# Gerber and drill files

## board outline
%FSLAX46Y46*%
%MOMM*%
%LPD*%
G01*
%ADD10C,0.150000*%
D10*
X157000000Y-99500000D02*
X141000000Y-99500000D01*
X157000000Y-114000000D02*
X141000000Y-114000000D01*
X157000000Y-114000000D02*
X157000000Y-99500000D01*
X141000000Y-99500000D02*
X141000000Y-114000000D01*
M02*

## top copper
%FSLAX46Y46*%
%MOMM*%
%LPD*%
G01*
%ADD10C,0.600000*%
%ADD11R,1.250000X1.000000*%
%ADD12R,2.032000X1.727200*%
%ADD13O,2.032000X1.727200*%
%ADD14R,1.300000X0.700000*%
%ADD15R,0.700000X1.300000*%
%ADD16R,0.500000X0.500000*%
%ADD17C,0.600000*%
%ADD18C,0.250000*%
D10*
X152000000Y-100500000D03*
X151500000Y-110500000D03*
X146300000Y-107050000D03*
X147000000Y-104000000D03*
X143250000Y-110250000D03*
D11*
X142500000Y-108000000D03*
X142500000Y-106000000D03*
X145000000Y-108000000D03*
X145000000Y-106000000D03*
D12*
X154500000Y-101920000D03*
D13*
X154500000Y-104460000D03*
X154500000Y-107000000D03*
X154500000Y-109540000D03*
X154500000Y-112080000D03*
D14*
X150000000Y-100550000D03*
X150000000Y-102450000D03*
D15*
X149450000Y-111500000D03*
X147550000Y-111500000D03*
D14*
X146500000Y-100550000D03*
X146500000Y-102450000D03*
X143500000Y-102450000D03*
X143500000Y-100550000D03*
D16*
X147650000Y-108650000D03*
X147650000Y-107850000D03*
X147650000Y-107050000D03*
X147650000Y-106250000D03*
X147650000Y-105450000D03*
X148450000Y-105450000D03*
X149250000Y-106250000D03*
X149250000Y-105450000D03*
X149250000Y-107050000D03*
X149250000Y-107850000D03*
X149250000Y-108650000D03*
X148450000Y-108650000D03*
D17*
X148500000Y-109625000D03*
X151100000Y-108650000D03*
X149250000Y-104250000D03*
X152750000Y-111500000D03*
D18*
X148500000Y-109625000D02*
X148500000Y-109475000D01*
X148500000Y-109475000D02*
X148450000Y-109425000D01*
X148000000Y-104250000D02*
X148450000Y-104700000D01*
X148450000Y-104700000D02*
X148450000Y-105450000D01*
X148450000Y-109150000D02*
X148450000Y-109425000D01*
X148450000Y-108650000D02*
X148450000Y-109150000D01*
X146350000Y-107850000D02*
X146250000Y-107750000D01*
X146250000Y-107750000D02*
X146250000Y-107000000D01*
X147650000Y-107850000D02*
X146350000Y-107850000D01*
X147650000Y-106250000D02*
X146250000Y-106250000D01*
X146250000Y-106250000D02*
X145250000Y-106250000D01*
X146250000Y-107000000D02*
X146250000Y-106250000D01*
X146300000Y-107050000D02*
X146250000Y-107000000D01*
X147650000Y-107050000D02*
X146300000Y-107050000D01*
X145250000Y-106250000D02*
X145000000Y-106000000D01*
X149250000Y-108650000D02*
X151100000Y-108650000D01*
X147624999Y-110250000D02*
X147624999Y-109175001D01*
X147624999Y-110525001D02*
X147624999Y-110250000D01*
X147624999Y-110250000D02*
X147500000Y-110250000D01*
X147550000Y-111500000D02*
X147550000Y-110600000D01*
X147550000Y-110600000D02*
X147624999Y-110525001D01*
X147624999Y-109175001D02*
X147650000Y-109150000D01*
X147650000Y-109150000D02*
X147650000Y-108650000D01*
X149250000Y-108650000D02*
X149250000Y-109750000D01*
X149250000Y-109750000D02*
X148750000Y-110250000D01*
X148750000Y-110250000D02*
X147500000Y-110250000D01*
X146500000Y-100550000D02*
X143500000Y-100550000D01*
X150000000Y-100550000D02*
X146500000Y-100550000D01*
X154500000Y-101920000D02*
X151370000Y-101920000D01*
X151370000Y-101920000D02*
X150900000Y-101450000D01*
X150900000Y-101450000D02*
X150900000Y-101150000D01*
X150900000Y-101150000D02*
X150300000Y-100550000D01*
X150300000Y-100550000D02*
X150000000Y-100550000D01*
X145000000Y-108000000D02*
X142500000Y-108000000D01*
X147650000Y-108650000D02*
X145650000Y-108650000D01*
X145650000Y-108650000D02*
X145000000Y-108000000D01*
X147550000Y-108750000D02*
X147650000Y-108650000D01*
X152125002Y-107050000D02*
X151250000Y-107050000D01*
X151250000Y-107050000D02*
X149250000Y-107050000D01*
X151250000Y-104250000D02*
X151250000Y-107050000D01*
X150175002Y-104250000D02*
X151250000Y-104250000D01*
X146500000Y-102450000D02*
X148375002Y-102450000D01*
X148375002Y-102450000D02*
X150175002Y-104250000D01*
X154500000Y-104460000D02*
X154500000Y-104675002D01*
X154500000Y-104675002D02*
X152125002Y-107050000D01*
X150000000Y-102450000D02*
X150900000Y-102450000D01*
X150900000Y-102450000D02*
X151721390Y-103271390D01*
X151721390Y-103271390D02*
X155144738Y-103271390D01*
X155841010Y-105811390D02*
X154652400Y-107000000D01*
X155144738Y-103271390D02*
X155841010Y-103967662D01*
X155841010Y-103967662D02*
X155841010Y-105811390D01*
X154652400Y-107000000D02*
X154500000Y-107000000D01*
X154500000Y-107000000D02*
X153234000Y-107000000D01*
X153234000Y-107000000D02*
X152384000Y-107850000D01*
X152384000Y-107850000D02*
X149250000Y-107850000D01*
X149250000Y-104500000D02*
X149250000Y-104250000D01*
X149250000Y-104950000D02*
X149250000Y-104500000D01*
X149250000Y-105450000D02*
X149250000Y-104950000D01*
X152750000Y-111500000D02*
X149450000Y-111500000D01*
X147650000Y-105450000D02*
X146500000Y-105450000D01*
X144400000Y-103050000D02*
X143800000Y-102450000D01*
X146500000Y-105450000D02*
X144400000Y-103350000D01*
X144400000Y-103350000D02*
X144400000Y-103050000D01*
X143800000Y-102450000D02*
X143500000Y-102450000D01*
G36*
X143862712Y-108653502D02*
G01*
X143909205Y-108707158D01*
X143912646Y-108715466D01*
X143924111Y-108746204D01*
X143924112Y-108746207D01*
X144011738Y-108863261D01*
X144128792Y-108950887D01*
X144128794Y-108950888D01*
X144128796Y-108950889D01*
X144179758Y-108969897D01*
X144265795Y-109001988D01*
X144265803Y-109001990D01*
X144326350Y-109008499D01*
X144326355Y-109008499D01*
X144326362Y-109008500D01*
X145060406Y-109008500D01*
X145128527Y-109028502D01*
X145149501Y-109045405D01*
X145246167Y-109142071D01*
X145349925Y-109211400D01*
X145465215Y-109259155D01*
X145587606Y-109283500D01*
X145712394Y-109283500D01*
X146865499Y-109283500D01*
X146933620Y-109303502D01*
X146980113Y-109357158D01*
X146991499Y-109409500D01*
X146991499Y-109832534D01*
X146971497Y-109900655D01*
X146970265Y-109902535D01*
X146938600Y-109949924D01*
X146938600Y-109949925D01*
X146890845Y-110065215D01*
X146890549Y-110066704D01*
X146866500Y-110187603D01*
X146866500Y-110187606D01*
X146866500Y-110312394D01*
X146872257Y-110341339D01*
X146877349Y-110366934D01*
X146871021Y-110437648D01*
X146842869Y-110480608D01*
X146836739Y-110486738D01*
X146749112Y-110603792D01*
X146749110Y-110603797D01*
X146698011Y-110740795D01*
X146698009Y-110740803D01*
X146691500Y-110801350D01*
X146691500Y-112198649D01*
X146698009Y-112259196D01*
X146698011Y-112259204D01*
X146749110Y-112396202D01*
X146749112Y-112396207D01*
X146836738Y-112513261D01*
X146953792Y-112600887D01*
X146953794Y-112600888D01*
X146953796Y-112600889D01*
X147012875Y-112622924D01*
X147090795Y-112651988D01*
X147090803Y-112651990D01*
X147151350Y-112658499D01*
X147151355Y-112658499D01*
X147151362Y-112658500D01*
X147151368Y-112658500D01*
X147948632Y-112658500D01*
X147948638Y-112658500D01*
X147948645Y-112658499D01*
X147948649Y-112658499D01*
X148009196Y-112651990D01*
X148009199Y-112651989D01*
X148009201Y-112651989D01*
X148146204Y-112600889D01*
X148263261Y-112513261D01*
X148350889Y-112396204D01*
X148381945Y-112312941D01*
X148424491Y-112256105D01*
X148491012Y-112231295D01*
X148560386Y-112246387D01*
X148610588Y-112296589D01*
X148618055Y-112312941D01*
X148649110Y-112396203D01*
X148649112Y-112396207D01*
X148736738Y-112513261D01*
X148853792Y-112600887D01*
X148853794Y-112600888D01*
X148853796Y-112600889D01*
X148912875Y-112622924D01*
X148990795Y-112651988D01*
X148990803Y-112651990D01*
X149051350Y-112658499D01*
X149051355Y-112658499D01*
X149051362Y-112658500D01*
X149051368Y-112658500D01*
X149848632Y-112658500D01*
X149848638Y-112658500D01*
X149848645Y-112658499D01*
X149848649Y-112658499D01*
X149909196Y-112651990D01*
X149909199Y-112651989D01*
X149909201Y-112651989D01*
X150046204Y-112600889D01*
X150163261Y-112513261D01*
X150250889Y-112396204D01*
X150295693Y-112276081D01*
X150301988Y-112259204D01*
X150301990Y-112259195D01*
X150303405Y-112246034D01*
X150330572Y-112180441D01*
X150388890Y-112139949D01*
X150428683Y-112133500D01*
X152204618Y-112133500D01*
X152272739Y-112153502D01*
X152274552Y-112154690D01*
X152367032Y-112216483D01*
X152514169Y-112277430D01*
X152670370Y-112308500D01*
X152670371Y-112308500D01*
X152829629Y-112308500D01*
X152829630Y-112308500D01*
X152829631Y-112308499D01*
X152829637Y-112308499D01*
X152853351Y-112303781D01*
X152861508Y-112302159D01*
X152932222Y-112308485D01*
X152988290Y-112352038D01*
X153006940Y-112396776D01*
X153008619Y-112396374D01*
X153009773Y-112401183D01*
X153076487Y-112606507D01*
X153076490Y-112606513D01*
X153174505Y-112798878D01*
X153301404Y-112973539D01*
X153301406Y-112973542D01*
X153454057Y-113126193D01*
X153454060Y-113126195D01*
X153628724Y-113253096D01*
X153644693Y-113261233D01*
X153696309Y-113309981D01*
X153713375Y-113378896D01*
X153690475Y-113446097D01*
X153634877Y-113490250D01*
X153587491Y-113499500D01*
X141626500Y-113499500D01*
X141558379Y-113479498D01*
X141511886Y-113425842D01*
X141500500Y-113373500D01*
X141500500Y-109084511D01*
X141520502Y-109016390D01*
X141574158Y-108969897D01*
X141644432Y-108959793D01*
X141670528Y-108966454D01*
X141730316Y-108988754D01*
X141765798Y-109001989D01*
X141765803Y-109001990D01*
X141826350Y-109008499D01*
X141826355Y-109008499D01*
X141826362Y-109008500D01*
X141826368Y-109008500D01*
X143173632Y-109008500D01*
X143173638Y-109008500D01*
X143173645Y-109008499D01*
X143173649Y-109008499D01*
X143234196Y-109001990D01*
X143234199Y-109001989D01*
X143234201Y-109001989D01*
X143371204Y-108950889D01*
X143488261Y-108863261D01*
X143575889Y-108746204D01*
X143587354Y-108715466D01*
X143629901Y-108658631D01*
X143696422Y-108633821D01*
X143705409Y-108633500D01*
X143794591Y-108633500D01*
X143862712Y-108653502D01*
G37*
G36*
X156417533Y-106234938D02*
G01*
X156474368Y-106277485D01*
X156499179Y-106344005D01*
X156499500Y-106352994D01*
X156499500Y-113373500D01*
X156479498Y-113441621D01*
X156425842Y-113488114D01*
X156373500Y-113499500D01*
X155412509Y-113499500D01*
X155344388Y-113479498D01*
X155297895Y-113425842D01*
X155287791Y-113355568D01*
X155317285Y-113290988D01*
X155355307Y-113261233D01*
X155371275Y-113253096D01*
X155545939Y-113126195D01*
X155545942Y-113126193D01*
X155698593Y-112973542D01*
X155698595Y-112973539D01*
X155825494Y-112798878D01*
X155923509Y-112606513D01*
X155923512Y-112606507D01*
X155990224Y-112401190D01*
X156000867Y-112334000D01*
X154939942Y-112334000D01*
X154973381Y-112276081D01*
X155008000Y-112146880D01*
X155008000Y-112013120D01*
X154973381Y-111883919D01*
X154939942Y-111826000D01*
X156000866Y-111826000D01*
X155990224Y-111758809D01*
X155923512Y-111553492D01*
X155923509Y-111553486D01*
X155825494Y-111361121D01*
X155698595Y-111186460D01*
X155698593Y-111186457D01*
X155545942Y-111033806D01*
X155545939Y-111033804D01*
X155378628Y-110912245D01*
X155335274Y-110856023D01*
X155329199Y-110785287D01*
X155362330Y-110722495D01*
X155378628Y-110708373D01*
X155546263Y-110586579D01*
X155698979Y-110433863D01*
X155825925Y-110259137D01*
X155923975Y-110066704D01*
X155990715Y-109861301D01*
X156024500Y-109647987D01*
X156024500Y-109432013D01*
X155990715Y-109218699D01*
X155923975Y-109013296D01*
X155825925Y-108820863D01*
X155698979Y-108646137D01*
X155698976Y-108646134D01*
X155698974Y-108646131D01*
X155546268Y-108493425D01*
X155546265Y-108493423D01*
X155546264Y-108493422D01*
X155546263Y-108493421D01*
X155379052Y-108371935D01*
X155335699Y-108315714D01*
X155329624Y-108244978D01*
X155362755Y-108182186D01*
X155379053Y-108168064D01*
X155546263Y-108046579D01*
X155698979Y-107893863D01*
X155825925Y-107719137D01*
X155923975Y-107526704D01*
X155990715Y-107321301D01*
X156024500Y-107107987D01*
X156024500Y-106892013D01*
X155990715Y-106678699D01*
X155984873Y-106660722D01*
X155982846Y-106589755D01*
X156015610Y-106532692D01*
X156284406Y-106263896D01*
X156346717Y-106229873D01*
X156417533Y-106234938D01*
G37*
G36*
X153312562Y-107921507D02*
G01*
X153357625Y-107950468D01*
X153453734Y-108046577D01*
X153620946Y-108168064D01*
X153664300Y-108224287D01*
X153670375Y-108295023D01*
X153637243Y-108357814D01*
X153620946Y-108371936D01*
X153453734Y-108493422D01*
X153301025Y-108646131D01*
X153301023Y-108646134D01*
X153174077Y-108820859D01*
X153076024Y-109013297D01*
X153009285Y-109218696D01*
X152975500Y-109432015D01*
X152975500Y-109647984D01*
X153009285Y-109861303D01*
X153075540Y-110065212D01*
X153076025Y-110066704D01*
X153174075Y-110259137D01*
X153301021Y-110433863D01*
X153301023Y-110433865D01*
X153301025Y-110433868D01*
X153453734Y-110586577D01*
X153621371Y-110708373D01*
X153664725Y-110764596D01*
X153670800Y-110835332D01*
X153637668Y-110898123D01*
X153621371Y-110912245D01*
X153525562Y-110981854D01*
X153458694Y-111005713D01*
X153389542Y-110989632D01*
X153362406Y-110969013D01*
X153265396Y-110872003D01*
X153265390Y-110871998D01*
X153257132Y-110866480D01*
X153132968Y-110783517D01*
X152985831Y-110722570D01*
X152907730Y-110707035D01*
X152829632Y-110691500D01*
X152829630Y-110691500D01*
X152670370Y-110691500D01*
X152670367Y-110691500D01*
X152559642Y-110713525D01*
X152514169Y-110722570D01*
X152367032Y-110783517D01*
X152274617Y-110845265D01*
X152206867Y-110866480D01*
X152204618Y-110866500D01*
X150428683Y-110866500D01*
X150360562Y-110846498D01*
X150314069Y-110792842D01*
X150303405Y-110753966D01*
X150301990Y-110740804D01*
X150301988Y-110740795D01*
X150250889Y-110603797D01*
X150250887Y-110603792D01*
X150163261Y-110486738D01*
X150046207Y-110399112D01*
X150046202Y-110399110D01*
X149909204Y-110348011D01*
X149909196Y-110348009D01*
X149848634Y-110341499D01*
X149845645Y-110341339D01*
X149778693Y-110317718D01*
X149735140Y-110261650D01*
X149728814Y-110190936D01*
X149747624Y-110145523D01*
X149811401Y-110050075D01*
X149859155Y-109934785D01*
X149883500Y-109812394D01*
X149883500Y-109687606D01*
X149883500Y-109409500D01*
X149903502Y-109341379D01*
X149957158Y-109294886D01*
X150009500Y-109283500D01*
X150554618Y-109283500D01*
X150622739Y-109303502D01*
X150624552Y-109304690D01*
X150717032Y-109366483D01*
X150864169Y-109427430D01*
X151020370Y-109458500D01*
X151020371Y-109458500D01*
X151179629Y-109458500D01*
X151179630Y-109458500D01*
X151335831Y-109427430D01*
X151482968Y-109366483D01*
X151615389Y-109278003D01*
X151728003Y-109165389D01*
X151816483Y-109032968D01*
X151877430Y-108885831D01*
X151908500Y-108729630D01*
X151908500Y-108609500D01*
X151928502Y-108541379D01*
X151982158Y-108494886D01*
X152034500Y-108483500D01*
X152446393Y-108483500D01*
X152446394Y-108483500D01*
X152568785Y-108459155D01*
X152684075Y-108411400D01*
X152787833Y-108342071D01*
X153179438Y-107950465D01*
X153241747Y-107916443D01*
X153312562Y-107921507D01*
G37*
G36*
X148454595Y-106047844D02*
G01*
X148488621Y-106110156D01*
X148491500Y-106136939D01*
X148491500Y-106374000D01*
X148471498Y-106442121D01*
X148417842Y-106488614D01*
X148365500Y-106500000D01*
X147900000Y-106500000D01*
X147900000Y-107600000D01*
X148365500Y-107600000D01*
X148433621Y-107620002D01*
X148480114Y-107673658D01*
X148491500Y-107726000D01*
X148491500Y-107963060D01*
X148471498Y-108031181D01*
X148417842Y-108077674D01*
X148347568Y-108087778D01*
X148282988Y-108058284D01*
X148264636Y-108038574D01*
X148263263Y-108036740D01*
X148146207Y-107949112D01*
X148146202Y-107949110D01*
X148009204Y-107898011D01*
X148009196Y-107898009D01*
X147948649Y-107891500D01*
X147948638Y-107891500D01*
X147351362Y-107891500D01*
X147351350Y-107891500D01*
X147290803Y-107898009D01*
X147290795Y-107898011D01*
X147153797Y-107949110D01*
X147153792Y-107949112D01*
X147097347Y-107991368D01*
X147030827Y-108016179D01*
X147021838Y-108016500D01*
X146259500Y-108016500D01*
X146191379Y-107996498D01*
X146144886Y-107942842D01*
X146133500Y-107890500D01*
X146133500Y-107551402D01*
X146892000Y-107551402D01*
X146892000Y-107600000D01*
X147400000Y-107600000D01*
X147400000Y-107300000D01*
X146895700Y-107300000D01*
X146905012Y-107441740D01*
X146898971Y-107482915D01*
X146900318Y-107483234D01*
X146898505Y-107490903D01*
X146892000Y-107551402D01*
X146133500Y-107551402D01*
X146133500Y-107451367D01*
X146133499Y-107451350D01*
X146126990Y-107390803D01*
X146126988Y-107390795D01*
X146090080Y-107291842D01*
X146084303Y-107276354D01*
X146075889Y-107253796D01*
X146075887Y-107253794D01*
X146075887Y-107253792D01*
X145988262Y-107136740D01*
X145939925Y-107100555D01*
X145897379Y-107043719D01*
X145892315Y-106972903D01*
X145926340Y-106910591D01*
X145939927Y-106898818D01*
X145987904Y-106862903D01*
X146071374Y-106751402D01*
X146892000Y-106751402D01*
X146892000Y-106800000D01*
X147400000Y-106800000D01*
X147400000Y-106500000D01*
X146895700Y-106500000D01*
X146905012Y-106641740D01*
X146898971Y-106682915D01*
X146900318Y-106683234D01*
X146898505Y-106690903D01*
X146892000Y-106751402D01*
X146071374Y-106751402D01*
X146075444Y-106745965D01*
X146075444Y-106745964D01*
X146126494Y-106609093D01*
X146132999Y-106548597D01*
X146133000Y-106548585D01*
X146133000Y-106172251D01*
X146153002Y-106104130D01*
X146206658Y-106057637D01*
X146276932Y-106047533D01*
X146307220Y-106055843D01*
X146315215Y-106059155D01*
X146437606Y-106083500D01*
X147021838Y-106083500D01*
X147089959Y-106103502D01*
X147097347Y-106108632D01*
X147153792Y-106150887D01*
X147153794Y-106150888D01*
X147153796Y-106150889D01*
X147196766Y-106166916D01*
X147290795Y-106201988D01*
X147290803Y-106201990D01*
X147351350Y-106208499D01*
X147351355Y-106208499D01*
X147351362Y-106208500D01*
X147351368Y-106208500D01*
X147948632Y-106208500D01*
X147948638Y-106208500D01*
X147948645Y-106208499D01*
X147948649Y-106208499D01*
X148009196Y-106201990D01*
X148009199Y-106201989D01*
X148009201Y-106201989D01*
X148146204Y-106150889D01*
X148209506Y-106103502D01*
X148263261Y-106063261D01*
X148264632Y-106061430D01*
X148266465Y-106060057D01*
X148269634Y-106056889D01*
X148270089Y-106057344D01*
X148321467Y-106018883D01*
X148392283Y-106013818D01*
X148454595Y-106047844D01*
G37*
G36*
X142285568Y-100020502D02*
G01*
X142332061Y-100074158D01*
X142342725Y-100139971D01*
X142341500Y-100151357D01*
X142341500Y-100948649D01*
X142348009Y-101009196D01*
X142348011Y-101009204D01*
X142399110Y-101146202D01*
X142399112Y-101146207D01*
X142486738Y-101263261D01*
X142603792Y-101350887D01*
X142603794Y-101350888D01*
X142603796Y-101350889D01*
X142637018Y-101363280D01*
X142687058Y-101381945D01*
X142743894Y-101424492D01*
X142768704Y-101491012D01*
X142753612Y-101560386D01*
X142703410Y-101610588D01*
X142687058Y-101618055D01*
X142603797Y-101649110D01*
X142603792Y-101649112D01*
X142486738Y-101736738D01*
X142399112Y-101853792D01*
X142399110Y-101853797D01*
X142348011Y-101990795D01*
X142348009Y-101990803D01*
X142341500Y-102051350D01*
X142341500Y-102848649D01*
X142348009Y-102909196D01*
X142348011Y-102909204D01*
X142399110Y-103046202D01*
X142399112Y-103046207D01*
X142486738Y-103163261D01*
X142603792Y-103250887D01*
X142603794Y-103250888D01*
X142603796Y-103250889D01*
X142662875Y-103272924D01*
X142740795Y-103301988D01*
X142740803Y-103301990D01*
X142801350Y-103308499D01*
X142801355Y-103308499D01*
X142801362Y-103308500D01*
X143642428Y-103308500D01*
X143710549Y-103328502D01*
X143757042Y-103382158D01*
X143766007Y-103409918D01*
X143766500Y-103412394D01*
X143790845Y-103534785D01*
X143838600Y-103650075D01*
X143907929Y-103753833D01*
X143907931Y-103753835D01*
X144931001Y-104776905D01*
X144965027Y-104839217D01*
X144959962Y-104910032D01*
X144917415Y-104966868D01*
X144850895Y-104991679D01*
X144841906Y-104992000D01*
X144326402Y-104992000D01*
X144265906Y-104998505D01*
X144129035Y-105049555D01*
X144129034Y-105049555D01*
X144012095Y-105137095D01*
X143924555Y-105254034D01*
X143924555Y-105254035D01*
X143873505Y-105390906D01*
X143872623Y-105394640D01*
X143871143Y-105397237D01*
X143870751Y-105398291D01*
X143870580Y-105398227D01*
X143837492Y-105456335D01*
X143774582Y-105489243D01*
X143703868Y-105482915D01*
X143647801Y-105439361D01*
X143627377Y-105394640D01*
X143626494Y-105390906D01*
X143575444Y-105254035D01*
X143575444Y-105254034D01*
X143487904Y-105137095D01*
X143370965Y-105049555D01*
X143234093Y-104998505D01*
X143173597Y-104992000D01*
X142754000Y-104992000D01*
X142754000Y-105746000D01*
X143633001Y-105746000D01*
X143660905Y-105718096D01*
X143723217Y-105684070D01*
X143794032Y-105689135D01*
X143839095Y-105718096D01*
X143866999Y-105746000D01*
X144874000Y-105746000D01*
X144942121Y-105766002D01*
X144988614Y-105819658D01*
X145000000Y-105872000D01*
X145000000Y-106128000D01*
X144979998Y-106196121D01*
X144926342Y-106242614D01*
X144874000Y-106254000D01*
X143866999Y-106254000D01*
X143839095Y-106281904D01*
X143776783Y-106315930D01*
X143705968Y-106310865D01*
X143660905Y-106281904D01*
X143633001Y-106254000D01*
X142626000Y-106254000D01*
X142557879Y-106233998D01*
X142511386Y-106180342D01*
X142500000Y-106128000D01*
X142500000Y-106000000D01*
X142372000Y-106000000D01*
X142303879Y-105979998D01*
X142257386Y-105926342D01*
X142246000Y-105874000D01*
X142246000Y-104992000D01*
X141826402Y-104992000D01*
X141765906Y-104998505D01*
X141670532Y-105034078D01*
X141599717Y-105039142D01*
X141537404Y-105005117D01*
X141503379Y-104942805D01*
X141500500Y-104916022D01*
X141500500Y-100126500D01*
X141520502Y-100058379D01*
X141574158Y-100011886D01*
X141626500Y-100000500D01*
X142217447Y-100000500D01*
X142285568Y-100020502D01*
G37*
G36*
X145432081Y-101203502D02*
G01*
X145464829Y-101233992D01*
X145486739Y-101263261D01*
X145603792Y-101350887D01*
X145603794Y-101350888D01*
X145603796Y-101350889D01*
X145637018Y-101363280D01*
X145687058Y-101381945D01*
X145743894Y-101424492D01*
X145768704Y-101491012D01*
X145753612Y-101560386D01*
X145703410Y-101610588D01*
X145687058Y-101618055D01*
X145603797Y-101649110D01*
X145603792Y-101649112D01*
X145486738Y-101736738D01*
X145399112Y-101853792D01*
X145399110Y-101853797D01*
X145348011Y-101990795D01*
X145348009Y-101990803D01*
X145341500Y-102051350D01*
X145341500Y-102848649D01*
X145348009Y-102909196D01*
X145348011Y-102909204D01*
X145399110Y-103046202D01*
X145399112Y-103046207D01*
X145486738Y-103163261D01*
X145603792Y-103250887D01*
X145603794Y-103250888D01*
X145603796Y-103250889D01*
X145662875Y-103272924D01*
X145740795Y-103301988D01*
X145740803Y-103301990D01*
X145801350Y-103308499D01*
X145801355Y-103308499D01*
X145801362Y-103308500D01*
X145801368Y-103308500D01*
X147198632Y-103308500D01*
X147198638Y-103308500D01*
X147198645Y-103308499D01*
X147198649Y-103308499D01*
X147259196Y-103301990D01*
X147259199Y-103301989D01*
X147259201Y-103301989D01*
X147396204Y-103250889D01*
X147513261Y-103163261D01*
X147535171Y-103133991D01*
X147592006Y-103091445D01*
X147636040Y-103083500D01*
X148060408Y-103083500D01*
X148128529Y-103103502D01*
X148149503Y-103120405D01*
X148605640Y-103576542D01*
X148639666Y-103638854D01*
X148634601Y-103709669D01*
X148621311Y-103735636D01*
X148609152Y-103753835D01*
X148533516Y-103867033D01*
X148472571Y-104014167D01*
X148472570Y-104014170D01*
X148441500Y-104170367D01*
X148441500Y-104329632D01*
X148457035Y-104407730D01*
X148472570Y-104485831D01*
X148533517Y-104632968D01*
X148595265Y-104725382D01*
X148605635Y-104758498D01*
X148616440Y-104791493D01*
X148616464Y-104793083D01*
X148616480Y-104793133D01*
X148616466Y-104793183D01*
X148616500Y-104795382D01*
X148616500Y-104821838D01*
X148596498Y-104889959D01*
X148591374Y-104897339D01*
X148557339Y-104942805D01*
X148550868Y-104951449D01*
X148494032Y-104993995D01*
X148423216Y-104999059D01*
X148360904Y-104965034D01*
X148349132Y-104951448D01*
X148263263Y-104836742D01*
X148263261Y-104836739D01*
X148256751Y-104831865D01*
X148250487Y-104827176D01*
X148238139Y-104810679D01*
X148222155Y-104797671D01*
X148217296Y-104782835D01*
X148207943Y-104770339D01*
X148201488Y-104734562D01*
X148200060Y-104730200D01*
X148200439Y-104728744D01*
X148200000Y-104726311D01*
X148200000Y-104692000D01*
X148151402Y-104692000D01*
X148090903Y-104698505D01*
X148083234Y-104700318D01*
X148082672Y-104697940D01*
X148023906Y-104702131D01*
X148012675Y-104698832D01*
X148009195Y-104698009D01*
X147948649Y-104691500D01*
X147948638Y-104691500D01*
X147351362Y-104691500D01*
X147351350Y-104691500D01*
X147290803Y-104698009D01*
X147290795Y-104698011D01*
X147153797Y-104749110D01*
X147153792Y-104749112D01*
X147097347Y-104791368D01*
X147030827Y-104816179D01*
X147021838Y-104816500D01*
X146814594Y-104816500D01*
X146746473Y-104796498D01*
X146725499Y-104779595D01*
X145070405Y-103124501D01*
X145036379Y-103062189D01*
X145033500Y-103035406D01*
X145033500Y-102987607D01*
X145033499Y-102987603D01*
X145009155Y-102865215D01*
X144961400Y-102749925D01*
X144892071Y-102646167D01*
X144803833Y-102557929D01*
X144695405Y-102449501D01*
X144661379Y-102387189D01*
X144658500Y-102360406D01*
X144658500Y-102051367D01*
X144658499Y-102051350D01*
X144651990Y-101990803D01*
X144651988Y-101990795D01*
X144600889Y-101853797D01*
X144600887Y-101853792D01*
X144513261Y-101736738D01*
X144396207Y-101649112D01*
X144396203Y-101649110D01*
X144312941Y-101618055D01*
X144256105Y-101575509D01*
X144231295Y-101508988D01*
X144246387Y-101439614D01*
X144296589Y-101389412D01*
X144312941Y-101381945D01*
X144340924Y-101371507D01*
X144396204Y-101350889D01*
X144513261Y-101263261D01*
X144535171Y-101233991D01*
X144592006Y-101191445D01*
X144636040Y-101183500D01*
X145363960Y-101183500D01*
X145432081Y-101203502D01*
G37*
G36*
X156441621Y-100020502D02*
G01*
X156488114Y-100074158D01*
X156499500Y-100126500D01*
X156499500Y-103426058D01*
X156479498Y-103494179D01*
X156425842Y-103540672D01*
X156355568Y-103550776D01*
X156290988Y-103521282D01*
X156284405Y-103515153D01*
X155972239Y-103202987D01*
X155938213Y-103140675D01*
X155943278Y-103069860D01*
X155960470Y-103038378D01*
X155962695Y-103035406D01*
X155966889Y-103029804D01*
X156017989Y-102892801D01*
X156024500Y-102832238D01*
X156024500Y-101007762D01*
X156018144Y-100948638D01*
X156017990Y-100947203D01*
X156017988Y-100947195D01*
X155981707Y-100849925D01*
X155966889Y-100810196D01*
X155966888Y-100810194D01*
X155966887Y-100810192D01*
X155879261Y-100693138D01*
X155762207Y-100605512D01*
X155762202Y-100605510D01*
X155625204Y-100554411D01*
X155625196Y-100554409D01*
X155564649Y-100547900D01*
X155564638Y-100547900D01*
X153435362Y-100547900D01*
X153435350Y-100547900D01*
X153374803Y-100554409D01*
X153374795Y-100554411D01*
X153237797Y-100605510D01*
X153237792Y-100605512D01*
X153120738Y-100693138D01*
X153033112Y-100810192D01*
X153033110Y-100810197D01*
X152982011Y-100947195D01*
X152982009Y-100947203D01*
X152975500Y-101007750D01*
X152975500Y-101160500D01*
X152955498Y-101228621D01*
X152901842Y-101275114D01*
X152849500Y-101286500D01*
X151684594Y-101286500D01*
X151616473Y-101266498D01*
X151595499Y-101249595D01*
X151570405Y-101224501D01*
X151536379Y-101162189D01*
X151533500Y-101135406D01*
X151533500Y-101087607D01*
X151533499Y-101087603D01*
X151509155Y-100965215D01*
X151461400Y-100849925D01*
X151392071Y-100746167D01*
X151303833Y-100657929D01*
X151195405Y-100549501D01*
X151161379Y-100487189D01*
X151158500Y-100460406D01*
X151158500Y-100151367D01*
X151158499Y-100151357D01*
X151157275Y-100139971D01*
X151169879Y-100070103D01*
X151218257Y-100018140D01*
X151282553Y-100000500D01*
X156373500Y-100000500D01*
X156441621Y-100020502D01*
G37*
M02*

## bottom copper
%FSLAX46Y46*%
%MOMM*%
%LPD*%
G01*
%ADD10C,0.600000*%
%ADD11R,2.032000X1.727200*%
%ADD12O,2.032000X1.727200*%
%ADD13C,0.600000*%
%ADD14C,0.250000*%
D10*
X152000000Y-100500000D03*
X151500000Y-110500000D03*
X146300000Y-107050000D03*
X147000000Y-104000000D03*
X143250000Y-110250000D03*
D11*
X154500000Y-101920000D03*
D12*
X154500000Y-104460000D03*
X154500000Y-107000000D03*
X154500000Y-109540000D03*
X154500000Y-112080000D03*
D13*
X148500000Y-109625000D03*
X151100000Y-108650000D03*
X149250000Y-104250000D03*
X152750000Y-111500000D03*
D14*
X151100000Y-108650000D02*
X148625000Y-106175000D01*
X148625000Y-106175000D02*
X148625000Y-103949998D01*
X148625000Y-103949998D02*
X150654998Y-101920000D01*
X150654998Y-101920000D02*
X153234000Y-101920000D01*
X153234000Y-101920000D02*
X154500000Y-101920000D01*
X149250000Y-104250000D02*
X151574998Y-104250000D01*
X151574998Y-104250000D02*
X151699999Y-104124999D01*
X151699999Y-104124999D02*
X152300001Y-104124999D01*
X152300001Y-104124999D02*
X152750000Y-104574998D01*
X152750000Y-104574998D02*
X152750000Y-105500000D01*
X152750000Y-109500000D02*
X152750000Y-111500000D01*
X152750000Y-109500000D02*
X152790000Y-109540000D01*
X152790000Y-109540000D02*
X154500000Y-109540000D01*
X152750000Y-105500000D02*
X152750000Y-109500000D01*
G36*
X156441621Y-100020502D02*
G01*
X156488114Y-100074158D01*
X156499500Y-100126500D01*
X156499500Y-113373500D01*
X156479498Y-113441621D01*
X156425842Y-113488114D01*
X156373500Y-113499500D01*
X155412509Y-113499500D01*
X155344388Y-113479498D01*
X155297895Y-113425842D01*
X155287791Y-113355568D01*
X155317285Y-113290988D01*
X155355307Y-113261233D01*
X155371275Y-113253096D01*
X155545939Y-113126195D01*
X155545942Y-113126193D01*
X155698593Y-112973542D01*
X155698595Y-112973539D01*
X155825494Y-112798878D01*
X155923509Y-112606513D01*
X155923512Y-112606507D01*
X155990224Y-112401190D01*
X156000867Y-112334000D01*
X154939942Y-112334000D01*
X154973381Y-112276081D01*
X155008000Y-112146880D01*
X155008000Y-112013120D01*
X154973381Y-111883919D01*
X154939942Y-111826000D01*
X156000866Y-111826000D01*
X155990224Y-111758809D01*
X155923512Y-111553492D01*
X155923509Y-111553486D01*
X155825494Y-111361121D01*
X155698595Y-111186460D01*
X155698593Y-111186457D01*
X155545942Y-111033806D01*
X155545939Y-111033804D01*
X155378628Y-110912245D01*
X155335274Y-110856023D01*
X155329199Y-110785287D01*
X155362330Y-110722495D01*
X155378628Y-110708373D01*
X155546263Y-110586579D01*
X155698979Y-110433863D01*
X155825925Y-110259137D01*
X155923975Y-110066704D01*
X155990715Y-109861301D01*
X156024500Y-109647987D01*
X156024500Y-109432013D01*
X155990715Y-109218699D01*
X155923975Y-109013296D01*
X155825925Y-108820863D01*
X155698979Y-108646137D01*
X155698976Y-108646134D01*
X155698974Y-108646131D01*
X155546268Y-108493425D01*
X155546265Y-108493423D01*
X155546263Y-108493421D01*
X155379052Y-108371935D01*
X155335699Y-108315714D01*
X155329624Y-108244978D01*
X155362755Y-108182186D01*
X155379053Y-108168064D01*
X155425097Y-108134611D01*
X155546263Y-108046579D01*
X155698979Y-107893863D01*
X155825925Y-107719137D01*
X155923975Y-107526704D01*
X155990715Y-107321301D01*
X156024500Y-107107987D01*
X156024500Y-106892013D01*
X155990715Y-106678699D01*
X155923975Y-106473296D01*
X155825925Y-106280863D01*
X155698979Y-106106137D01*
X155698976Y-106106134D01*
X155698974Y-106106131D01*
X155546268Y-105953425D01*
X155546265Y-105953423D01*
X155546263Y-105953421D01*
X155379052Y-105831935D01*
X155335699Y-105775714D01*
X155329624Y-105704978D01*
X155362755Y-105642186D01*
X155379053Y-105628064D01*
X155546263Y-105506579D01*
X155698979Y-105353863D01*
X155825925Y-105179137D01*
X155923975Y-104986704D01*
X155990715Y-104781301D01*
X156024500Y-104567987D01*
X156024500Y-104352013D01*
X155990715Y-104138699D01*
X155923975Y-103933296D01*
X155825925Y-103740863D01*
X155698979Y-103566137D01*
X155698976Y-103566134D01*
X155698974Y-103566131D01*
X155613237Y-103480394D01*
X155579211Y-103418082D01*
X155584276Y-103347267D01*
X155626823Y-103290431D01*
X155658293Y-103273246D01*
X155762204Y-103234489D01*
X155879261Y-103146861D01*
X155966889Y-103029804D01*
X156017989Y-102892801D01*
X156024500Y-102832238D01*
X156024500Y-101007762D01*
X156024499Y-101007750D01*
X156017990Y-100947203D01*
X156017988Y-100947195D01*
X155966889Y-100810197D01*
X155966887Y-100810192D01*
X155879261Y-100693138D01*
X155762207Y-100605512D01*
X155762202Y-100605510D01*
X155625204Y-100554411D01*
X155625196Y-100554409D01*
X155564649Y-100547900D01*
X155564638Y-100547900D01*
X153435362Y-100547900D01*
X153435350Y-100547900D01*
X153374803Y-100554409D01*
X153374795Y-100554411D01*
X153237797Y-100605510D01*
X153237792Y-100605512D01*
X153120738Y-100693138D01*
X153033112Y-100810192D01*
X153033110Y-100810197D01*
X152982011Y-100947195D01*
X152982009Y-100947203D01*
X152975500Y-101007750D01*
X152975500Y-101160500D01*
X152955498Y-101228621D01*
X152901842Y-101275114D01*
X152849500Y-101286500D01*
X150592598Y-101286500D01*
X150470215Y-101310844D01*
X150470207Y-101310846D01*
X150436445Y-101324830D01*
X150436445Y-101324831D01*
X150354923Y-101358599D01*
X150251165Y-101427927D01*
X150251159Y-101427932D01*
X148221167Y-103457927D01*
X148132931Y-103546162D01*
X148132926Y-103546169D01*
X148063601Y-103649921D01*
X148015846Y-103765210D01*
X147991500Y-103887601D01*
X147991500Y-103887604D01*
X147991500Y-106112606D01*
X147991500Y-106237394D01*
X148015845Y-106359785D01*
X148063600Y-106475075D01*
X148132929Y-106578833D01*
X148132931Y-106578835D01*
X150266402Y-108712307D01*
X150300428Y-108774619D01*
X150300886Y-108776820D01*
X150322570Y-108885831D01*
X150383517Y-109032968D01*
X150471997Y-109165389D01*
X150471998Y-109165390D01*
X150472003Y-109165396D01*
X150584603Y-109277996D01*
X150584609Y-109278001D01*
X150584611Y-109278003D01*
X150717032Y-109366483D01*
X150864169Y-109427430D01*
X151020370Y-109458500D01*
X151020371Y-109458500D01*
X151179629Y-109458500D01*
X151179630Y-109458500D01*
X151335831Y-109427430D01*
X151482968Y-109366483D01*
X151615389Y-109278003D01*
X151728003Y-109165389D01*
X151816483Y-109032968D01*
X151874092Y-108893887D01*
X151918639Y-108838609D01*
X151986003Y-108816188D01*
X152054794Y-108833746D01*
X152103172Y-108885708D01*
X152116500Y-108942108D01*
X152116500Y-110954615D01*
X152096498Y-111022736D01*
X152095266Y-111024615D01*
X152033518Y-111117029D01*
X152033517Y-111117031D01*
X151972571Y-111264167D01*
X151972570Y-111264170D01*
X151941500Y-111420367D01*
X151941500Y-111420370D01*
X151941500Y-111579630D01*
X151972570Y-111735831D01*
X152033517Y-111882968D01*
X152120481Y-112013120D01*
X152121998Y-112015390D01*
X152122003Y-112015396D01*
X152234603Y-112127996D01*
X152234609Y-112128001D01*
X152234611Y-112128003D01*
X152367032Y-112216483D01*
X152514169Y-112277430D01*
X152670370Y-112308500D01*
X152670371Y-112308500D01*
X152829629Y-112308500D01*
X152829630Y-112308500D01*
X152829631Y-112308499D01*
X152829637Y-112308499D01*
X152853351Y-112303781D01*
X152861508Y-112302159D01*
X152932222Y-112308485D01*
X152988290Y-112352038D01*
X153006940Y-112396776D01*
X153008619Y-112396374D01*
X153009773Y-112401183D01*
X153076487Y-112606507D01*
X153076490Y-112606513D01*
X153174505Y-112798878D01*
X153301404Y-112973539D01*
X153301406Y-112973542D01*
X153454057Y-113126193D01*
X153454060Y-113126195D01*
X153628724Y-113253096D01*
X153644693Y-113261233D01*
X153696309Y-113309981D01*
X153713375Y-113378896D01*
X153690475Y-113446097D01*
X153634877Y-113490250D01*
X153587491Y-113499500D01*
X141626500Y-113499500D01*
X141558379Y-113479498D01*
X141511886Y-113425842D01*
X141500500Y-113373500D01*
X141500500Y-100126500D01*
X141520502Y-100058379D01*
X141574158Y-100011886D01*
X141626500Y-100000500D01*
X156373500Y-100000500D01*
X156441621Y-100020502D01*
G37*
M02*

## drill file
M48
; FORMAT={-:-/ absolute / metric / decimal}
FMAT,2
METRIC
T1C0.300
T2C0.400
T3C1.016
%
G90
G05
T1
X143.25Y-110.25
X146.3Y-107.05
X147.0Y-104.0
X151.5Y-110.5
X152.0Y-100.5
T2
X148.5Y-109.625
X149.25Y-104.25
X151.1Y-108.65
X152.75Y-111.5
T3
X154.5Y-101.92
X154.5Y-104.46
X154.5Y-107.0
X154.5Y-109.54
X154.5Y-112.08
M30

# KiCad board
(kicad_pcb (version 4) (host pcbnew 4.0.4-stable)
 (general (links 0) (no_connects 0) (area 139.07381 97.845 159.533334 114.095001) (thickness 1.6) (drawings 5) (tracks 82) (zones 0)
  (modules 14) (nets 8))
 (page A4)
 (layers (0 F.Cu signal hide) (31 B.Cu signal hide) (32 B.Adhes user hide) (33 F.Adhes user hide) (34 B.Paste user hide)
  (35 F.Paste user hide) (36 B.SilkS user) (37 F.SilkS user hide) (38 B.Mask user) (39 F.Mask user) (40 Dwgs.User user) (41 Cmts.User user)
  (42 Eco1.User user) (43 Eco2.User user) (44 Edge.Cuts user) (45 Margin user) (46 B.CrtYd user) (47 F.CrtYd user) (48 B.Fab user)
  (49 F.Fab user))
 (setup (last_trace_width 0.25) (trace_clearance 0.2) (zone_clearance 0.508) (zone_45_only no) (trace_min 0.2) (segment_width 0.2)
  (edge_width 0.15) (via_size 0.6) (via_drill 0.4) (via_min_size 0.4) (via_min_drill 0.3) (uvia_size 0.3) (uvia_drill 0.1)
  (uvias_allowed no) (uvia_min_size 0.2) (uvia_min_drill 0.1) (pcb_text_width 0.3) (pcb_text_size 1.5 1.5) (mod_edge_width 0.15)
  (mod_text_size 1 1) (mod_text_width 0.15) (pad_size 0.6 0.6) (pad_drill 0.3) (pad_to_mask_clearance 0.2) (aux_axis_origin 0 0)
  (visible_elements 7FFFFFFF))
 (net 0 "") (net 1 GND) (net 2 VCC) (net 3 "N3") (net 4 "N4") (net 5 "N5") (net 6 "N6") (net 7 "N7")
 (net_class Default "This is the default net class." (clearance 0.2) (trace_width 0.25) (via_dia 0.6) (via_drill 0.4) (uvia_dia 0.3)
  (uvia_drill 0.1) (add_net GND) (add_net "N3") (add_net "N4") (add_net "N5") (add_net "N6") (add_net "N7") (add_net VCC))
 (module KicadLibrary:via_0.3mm (layer F.Cu) (at 152 100.5)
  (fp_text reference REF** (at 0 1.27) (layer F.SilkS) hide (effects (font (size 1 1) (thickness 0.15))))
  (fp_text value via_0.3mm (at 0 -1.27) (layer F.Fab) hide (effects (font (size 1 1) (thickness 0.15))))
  (pad 1 thru_hole circle (at 0 0) (size 0.6 0.6) (drill 0.3) (layers *.Cu) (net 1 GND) (zone_connect 2)))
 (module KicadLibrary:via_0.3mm (layer F.Cu) (at 151.5 110.5)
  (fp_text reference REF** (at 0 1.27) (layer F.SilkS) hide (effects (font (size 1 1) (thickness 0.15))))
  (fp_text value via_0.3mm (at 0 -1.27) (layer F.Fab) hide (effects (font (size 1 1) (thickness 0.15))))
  (pad 1 thru_hole circle (at 0 0) (size 0.6 0.6) (drill 0.3) (layers *.Cu) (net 1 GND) (zone_connect 2)))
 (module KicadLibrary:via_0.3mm (layer F.Cu) (at 146.3 107.05)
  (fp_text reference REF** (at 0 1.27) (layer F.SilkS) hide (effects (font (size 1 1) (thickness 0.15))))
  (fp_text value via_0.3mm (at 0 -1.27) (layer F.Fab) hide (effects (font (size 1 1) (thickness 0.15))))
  (pad 1 thru_hole circle (at 0 0) (size 0.6 0.6) (drill 0.3) (layers *.Cu) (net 1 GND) (zone_connect 2)))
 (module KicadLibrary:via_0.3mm (layer F.Cu) (at 147 104)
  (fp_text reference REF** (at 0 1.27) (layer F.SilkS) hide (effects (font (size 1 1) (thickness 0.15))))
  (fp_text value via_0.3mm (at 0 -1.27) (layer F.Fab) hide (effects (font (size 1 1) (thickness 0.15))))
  (pad 1 thru_hole circle (at 0 0) (size 0.6 0.6) (drill 0.3) (layers *.Cu) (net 1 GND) (zone_connect 2)))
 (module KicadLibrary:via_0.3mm (layer F.Cu) (at 143.25 110.25)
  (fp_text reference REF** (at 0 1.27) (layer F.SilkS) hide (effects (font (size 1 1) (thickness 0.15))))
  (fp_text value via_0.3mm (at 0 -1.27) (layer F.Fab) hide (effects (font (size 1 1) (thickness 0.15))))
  (pad 1 thru_hole circle (at 0 0) (size 0.6 0.6) (drill 0.3) (layers *.Cu) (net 1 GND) (zone_connect 2)))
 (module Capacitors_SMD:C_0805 (layer F.Cu) (at 142.5 107 90)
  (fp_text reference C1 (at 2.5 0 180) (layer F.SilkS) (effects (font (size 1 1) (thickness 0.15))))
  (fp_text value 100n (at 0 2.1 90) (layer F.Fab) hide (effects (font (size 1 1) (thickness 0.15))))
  (pad 1 smd rect (at -1 0 90) (size 1 1.25) (layers F.Cu F.Paste F.Mask) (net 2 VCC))
  (pad 2 smd rect (at 1 0 90) (size 1 1.25) (layers F.Cu F.Paste F.Mask) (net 1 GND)))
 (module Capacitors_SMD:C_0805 (layer F.Cu) (at 145 107 90)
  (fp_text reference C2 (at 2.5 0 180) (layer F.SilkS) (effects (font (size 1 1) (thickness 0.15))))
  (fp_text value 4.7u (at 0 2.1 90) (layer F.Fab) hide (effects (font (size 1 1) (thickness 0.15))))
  (pad 1 smd rect (at -1 0 90) (size 1 1.25) (layers F.Cu F.Paste F.Mask) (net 2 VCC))
  (pad 2 smd rect (at 1 0 90) (size 1 1.25) (layers F.Cu F.Paste F.Mask) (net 1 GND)))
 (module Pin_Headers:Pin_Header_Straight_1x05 (layer F.Cu) (at 154.5 101.92)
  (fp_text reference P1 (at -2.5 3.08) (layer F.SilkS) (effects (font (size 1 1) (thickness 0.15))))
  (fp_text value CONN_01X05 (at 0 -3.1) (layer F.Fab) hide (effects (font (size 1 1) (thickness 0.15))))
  (pad 1 thru_hole rect (at 0 0) (size 2.032 1.7272) (drill 1.016) (layers *.Cu *.Mask) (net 2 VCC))
  (pad 2 thru_hole oval (at 0 2.54) (size 2.032 1.7272) (drill 1.016) (layers *.Cu *.Mask) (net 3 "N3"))
  (pad 3 thru_hole oval (at 0 5.08) (size 2.032 1.7272) (drill 1.016) (layers *.Cu *.Mask) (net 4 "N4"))
  (pad 4 thru_hole oval (at 0 7.62) (size 2.032 1.7272) (drill 1.016) (layers *.Cu *.Mask) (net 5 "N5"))
  (pad 5 thru_hole oval (at 0 10.16) (size 2.032 1.7272) (drill 1.016) (layers *.Cu *.Mask) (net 1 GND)))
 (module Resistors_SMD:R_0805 (layer F.Cu) (at 150 101.5 270)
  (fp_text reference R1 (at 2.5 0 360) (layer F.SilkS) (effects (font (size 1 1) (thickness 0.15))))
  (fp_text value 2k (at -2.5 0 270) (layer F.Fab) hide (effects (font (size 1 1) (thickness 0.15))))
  (pad 1 smd rect (at -0.95 0 270) (size 0.7 1.3) (layers F.Cu F.Paste F.Mask) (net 2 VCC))
  (pad 2 smd rect (at 0.95 0 270) (size 0.7 1.3) (layers F.Cu F.Paste F.Mask) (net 4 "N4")))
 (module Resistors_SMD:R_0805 (layer F.Cu) (at 148.5 111.5 180)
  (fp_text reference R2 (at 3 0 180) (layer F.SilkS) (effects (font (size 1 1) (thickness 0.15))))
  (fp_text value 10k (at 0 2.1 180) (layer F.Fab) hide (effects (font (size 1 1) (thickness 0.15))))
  (pad 1 smd rect (at -0.95 0 180) (size 0.7 1.3) (layers F.Cu F.Paste F.Mask) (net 5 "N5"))
  (pad 2 smd rect (at 0.95 0 180) (size 0.7 1.3) (layers F.Cu F.Paste F.Mask) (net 2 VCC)))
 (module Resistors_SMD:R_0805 (layer F.Cu) (at 146.5 101.5 270)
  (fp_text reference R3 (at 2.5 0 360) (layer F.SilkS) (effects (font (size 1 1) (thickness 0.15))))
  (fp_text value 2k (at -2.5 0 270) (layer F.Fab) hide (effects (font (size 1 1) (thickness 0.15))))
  (pad 1 smd rect (at -0.95 0 270) (size 0.7 1.3) (layers F.Cu F.Paste F.Mask) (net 2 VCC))
  (pad 2 smd rect (at 0.95 0 270) (size 0.7 1.3) (layers F.Cu F.Paste F.Mask) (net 3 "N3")))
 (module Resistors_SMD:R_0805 (layer F.Cu) (at 143.5 101.5 90)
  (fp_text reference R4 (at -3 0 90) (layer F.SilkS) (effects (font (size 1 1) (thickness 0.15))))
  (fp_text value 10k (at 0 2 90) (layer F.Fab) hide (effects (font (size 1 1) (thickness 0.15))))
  (pad 1 smd rect (at -0.95 0 90) (size 0.7 1.3) (layers F.Cu F.Paste F.Mask) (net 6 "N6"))
  (pad 2 smd rect (at 0.95 0 90) (size 0.7 1.3) (layers F.Cu F.Paste F.Mask) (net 2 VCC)))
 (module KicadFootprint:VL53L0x (layer F.Cu) (at 148.5 107 90)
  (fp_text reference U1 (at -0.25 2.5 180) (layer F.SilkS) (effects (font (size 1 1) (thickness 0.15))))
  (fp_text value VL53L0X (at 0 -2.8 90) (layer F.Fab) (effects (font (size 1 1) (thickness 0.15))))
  (pad 1 smd rect (at -1.65 -0.85 90) (size 0.5 0.5) (layers F.Cu F.Paste F.Mask) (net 2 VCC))
  (pad 2 smd rect (at -0.85 -0.85 90) (size 0.5 0.5) (layers F.Cu F.Paste F.Mask) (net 1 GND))
  (pad 3 smd rect (at -0.05 -0.85 90) (size 0.5 0.5) (layers F.Cu F.Paste F.Mask) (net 1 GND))
  (pad 4 smd rect (at 0.75 -0.85 90) (size 0.5 0.5) (layers F.Cu F.Paste F.Mask) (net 1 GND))
  (pad 5 smd rect (at 1.55 -0.85 90) (size 0.5 0.5) (layers F.Cu F.Paste F.Mask) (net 6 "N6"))
  (pad 6 smd rect (at 1.55 -0.05 90) (size 0.5 0.5) (layers F.Cu F.Paste F.Mask) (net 1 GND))
  (pad 8 smd rect (at 0.75 0.75 90) (size 0.5 0.5) (layers F.Cu F.Paste F.Mask) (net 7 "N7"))
  (pad 7 smd rect (at 1.55 0.75 90) (size 0.5 0.5) (layers F.Cu F.Paste F.Mask) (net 5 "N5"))
  (pad 9 smd rect (at -0.05 0.75 90) (size 0.5 0.5) (layers F.Cu F.Paste F.Mask) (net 3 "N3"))
  (pad 10 smd rect (at -0.85 0.75 90) (size 0.5 0.5) (layers F.Cu F.Paste F.Mask) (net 4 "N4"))
  (pad 11 smd rect (at -1.65 0.75 90) (size 0.5 0.5) (layers F.Cu F.Paste F.Mask) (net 2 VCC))
  (pad 12 smd rect (at -1.65 -0.05 90) (size 0.5 0.5) (layers F.Cu F.Paste F.Mask) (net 1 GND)))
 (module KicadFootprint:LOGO (layer B.Cu) (at 146.8 108.4 180)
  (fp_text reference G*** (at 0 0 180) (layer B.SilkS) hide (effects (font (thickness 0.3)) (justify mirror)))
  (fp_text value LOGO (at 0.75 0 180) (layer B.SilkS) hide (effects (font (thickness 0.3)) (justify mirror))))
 (gr_line (start 157 99.5) (end 141 99.5) (layer Edge.Cuts) (width 0.15))
 (gr_line (start 157 114) (end 141 114) (layer Edge.Cuts) (width 0.15))
 (gr_line (start 157 114) (end 157 99.5) (layer Edge.Cuts) (width 0.15))
 (gr_line (start 141 99.5) (end 141 114) (layer Edge.Cuts) (width 0.15))
 (segment (start 148.5 109.625) (end 148.5 109.475) (width 0.25) (layer F.Cu) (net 1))
 (segment (start 148.5 109.475) (end 148.45 109.425) (width 0.25) (layer F.Cu) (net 1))
 (segment (start 148 104.25) (end 148.45 104.7) (width 0.25) (layer F.Cu) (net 1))
 (segment (start 148.45 104.7) (end 148.45 105.45) (width 0.25) (layer F.Cu) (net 1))
 (segment (start 148.45 109.15) (end 148.45 109.425) (width 0.25) (layer F.Cu) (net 1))
 (via (at 148.5 109.625) (size 0.6) (drill 0.4) (layers F.Cu B.Cu) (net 1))
 (segment (start 148.45 108.65) (end 148.45 109.15) (width 0.25) (layer F.Cu) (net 1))
 (segment (start 146.35 107.85) (end 146.25 107.75) (width 0.25) (layer F.Cu) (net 1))
 (segment (start 146.25 107.75) (end 146.25 107) (width 0.25) (layer F.Cu) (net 1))
 (segment (start 147.65 107.85) (end 146.35 107.85) (width 0.25) (layer F.Cu) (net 1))
 (segment (start 147.65 106.25) (end 146.25 106.25) (width 0.25) (layer F.Cu) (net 1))
 (segment (start 146.25 106.25) (end 145.25 106.25) (width 0.25) (layer F.Cu) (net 1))
 (segment (start 146.25 107) (end 146.25 106.25) (width 0.25) (layer F.Cu) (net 1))
 (segment (start 146.3 107.05) (end 146.25 107) (width 0.25) (layer F.Cu) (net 1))
 (segment (start 147.65 107.05) (end 146.3 107.05) (width 0.25) (layer F.Cu) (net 1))
 (segment (start 145.25 106.25) (end 145 106) (width 0.25) (layer F.Cu) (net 1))
 (segment (start 151.1 108.65) (end 148.625 106.175) (width 0.25) (layer B.Cu) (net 2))
 (segment (start 148.625 106.175) (end 148.625 103.949998) (width 0.25) (layer B.Cu) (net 2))
 (segment (start 148.625 103.949998) (end 150.654998 101.92) (width 0.25) (layer B.Cu) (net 2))
 (segment (start 150.654998 101.92) (end 153.234 101.92) (width 0.25) (layer B.Cu) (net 2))
 (segment (start 153.234 101.92) (end 154.5 101.92) (width 0.25) (layer B.Cu) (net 2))
 (via (at 151.1 108.65) (size 0.6) (drill 0.4) (layers F.Cu B.Cu) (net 2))
 (segment (start 149.25 108.65) (end 151.1 108.65) (width 0.25) (layer F.Cu) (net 2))
 (segment (start 147.624999 110.25) (end 147.624999 109.175001) (width 0.25) (layer F.Cu) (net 2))
 (segment (start 147.624999 110.525001) (end 147.624999 110.25) (width 0.25) (layer F.Cu) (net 2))
 (segment (start 147.624999 110.25) (end 147.5 110.25) (width 0.25) (layer F.Cu) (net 2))
 (segment (start 147.55 111.5) (end 147.55 110.6) (width 0.25) (layer F.Cu) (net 2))
 (segment (start 147.55 110.6) (end 147.624999 110.525001) (width 0.25) (layer F.Cu) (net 2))
 (segment (start 147.624999 109.175001) (end 147.65 109.15) (width 0.25) (layer F.Cu) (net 2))
 (segment (start 147.65 109.15) (end 147.65 108.65) (width 0.25) (layer F.Cu) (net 2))
 (segment (start 149.25 108.65) (end 149.25 109.75) (width 0.25) (layer F.Cu) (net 2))
 (segment (start 149.25 109.75) (end 148.75 110.25) (width 0.25) (layer F.Cu) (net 2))
 (segment (start 148.75 110.25) (end 147.5 110.25) (width 0.25) (layer F.Cu) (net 2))
 (segment (start 146.5 100.55) (end 143.5 100.55) (width 0.25) (layer F.Cu) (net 2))
 (segment (start 150 100.55) (end 146.5 100.55) (width 0.25) (layer F.Cu) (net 2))
 (segment (start 154.5 101.92) (end 151.37 101.92) (width 0.25) (layer F.Cu) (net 2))
 (segment (start 151.37 101.92) (end 150.9 101.45) (width 0.25) (layer F.Cu) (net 2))
 (segment (start 150.9 101.45) (end 150.9 101.15) (width 0.25) (layer F.Cu) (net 2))
 (segment (start 150.9 101.15) (end 150.3 100.55) (width 0.25) (layer F.Cu) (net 2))
 (segment (start 150.3 100.55) (end 150 100.55) (width 0.25) (layer F.Cu) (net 2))
 (segment (start 145 108) (end 142.5 108) (width 0.25) (layer F.Cu) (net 2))
 (segment (start 147.65 108.65) (end 145.65 108.65) (width 0.25) (layer F.Cu) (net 2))
 (segment (start 145.65 108.65) (end 145 108) (width 0.25) (layer F.Cu) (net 2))
 (segment (start 147.55 108.75) (end 147.65 108.65) (width 0.25) (layer F.Cu) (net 2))
 (segment (start 152.125002 107.05) (end 151.25 107.05) (width 0.25) (layer F.Cu) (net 3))
 (segment (start 151.25 107.05) (end 149.25 107.05) (width 0.25) (layer F.Cu) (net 3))
 (segment (start 151.25 104.25) (end 151.25 107.05) (width 0.25) (layer F.Cu) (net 3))
 (segment (start 150.175002 104.25) (end 151.25 104.25) (width 0.25) (layer F.Cu) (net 3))
 (segment (start 146.5 102.45) (end 148.375002 102.45) (width 0.25) (layer F.Cu) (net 3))
 (segment (start 148.375002 102.45) (end 150.175002 104.25) (width 0.25) (layer F.Cu) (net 3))
 (segment (start 154.5 104.46) (end 154.5 104.675002) (width 0.25) (layer F.Cu) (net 3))
 (segment (start 154.5 104.675002) (end 152.125002 107.05) (width 0.25) (layer F.Cu) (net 3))
 (segment (start 150 102.45) (end 150.9 102.45) (width 0.25) (layer F.Cu) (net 4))
 (segment (start 150.9 102.45) (end 151.72139 103.27139) (width 0.25) (layer F.Cu) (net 4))
 (segment (start 151.72139 103.27139) (end 155.144738 103.27139) (width 0.25) (layer F.Cu) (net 4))
 (segment (start 155.84101 105.81139) (end 154.6524 107) (width 0.25) (layer F.Cu) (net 4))
 (segment (start 155.144738 103.27139) (end 155.84101 103.967662) (width 0.25) (layer F.Cu) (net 4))
 (segment (start 155.84101 103.967662) (end 155.84101 105.81139) (width 0.25) (layer F.Cu) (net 4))
 (segment (start 154.6524 107) (end 154.5 107) (width 0.25) (layer F.Cu) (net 4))
 (segment (start 154.5 107) (end 153.234 107) (width 0.25) (layer F.Cu) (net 4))
 (segment (start 153.234 107) (end 152.384 107.85) (width 0.25) (layer F.Cu) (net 4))
 (segment (start 152.384 107.85) (end 149.25 107.85) (width 0.25) (layer F.Cu) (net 4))
 (segment (start 149.25 104.25) (end 151.574998 104.25) (width 0.25) (layer B.Cu) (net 5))
 (segment (start 151.574998 104.25) (end 151.699999 104.124999) (width 0.25) (layer B.Cu) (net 5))
 (segment (start 151.699999 104.124999) (end 152.300001 104.124999) (width 0.25) (layer B.Cu) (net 5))
 (segment (start 152.300001 104.124999) (end 152.75 104.574998) (width 0.25) (layer B.Cu) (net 5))
 (segment (start 152.75 104.574998) (end 152.75 105.5) (width 0.25) (layer B.Cu) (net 5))
 (segment (start 149.25 104.5) (end 149.25 104.25) (width 0.25) (layer F.Cu) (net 5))
 (via (at 149.25 104.25) (size 0.6) (drill 0.4) (layers F.Cu B.Cu) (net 5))
 (segment (start 149.25 104.95) (end 149.25 104.5) (width 0.25) (layer F.Cu) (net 5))
 (segment (start 149.25 105.45) (end 149.25 104.95) (width 0.25) (layer F.Cu) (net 5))
 (segment (start 152.75 111.5) (end 149.45 111.5) (width 0.25) (layer F.Cu) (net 5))
 (via (at 152.75 111.5) (size 0.6) (drill 0.4) (layers F.Cu B.Cu) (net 5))
 (segment (start 152.75 109.5) (end 152.75 111.5) (width 0.25) (layer B.Cu) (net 5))
 (segment (start 152.75 109.5) (end 152.79 109.54) (width 0.25) (layer B.Cu) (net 5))
 (segment (start 152.79 109.54) (end 154.5 109.54) (width 0.25) (layer B.Cu) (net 5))
 (segment (start 152.75 105.5) (end 152.75 109.5) (width 0.25) (layer B.Cu) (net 5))
 (segment (start 147.65 105.45) (end 146.5 105.45) (width 0.25) (layer F.Cu) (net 6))
 (segment (start 144.4 103.05) (end 143.8 102.45) (width 0.25) (layer F.Cu) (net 6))
 (segment (start 146.5 105.45) (end 144.4 103.35) (width 0.25) (layer F.Cu) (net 6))
 (segment (start 144.4 103.35) (end 144.4 103.05) (width 0.25) (layer F.Cu) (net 6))
 (segment (start 143.8 102.45) (end 143.5 102.45) (width 0.25) (layer F.Cu) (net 6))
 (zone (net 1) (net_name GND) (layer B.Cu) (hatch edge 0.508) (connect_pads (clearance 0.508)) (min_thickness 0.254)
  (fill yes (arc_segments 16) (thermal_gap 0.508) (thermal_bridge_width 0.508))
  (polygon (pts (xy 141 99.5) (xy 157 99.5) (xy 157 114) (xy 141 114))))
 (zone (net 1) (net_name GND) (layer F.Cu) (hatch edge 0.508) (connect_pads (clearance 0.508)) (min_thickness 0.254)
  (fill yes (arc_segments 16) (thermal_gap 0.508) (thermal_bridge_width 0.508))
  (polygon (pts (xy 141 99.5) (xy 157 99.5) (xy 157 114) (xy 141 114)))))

